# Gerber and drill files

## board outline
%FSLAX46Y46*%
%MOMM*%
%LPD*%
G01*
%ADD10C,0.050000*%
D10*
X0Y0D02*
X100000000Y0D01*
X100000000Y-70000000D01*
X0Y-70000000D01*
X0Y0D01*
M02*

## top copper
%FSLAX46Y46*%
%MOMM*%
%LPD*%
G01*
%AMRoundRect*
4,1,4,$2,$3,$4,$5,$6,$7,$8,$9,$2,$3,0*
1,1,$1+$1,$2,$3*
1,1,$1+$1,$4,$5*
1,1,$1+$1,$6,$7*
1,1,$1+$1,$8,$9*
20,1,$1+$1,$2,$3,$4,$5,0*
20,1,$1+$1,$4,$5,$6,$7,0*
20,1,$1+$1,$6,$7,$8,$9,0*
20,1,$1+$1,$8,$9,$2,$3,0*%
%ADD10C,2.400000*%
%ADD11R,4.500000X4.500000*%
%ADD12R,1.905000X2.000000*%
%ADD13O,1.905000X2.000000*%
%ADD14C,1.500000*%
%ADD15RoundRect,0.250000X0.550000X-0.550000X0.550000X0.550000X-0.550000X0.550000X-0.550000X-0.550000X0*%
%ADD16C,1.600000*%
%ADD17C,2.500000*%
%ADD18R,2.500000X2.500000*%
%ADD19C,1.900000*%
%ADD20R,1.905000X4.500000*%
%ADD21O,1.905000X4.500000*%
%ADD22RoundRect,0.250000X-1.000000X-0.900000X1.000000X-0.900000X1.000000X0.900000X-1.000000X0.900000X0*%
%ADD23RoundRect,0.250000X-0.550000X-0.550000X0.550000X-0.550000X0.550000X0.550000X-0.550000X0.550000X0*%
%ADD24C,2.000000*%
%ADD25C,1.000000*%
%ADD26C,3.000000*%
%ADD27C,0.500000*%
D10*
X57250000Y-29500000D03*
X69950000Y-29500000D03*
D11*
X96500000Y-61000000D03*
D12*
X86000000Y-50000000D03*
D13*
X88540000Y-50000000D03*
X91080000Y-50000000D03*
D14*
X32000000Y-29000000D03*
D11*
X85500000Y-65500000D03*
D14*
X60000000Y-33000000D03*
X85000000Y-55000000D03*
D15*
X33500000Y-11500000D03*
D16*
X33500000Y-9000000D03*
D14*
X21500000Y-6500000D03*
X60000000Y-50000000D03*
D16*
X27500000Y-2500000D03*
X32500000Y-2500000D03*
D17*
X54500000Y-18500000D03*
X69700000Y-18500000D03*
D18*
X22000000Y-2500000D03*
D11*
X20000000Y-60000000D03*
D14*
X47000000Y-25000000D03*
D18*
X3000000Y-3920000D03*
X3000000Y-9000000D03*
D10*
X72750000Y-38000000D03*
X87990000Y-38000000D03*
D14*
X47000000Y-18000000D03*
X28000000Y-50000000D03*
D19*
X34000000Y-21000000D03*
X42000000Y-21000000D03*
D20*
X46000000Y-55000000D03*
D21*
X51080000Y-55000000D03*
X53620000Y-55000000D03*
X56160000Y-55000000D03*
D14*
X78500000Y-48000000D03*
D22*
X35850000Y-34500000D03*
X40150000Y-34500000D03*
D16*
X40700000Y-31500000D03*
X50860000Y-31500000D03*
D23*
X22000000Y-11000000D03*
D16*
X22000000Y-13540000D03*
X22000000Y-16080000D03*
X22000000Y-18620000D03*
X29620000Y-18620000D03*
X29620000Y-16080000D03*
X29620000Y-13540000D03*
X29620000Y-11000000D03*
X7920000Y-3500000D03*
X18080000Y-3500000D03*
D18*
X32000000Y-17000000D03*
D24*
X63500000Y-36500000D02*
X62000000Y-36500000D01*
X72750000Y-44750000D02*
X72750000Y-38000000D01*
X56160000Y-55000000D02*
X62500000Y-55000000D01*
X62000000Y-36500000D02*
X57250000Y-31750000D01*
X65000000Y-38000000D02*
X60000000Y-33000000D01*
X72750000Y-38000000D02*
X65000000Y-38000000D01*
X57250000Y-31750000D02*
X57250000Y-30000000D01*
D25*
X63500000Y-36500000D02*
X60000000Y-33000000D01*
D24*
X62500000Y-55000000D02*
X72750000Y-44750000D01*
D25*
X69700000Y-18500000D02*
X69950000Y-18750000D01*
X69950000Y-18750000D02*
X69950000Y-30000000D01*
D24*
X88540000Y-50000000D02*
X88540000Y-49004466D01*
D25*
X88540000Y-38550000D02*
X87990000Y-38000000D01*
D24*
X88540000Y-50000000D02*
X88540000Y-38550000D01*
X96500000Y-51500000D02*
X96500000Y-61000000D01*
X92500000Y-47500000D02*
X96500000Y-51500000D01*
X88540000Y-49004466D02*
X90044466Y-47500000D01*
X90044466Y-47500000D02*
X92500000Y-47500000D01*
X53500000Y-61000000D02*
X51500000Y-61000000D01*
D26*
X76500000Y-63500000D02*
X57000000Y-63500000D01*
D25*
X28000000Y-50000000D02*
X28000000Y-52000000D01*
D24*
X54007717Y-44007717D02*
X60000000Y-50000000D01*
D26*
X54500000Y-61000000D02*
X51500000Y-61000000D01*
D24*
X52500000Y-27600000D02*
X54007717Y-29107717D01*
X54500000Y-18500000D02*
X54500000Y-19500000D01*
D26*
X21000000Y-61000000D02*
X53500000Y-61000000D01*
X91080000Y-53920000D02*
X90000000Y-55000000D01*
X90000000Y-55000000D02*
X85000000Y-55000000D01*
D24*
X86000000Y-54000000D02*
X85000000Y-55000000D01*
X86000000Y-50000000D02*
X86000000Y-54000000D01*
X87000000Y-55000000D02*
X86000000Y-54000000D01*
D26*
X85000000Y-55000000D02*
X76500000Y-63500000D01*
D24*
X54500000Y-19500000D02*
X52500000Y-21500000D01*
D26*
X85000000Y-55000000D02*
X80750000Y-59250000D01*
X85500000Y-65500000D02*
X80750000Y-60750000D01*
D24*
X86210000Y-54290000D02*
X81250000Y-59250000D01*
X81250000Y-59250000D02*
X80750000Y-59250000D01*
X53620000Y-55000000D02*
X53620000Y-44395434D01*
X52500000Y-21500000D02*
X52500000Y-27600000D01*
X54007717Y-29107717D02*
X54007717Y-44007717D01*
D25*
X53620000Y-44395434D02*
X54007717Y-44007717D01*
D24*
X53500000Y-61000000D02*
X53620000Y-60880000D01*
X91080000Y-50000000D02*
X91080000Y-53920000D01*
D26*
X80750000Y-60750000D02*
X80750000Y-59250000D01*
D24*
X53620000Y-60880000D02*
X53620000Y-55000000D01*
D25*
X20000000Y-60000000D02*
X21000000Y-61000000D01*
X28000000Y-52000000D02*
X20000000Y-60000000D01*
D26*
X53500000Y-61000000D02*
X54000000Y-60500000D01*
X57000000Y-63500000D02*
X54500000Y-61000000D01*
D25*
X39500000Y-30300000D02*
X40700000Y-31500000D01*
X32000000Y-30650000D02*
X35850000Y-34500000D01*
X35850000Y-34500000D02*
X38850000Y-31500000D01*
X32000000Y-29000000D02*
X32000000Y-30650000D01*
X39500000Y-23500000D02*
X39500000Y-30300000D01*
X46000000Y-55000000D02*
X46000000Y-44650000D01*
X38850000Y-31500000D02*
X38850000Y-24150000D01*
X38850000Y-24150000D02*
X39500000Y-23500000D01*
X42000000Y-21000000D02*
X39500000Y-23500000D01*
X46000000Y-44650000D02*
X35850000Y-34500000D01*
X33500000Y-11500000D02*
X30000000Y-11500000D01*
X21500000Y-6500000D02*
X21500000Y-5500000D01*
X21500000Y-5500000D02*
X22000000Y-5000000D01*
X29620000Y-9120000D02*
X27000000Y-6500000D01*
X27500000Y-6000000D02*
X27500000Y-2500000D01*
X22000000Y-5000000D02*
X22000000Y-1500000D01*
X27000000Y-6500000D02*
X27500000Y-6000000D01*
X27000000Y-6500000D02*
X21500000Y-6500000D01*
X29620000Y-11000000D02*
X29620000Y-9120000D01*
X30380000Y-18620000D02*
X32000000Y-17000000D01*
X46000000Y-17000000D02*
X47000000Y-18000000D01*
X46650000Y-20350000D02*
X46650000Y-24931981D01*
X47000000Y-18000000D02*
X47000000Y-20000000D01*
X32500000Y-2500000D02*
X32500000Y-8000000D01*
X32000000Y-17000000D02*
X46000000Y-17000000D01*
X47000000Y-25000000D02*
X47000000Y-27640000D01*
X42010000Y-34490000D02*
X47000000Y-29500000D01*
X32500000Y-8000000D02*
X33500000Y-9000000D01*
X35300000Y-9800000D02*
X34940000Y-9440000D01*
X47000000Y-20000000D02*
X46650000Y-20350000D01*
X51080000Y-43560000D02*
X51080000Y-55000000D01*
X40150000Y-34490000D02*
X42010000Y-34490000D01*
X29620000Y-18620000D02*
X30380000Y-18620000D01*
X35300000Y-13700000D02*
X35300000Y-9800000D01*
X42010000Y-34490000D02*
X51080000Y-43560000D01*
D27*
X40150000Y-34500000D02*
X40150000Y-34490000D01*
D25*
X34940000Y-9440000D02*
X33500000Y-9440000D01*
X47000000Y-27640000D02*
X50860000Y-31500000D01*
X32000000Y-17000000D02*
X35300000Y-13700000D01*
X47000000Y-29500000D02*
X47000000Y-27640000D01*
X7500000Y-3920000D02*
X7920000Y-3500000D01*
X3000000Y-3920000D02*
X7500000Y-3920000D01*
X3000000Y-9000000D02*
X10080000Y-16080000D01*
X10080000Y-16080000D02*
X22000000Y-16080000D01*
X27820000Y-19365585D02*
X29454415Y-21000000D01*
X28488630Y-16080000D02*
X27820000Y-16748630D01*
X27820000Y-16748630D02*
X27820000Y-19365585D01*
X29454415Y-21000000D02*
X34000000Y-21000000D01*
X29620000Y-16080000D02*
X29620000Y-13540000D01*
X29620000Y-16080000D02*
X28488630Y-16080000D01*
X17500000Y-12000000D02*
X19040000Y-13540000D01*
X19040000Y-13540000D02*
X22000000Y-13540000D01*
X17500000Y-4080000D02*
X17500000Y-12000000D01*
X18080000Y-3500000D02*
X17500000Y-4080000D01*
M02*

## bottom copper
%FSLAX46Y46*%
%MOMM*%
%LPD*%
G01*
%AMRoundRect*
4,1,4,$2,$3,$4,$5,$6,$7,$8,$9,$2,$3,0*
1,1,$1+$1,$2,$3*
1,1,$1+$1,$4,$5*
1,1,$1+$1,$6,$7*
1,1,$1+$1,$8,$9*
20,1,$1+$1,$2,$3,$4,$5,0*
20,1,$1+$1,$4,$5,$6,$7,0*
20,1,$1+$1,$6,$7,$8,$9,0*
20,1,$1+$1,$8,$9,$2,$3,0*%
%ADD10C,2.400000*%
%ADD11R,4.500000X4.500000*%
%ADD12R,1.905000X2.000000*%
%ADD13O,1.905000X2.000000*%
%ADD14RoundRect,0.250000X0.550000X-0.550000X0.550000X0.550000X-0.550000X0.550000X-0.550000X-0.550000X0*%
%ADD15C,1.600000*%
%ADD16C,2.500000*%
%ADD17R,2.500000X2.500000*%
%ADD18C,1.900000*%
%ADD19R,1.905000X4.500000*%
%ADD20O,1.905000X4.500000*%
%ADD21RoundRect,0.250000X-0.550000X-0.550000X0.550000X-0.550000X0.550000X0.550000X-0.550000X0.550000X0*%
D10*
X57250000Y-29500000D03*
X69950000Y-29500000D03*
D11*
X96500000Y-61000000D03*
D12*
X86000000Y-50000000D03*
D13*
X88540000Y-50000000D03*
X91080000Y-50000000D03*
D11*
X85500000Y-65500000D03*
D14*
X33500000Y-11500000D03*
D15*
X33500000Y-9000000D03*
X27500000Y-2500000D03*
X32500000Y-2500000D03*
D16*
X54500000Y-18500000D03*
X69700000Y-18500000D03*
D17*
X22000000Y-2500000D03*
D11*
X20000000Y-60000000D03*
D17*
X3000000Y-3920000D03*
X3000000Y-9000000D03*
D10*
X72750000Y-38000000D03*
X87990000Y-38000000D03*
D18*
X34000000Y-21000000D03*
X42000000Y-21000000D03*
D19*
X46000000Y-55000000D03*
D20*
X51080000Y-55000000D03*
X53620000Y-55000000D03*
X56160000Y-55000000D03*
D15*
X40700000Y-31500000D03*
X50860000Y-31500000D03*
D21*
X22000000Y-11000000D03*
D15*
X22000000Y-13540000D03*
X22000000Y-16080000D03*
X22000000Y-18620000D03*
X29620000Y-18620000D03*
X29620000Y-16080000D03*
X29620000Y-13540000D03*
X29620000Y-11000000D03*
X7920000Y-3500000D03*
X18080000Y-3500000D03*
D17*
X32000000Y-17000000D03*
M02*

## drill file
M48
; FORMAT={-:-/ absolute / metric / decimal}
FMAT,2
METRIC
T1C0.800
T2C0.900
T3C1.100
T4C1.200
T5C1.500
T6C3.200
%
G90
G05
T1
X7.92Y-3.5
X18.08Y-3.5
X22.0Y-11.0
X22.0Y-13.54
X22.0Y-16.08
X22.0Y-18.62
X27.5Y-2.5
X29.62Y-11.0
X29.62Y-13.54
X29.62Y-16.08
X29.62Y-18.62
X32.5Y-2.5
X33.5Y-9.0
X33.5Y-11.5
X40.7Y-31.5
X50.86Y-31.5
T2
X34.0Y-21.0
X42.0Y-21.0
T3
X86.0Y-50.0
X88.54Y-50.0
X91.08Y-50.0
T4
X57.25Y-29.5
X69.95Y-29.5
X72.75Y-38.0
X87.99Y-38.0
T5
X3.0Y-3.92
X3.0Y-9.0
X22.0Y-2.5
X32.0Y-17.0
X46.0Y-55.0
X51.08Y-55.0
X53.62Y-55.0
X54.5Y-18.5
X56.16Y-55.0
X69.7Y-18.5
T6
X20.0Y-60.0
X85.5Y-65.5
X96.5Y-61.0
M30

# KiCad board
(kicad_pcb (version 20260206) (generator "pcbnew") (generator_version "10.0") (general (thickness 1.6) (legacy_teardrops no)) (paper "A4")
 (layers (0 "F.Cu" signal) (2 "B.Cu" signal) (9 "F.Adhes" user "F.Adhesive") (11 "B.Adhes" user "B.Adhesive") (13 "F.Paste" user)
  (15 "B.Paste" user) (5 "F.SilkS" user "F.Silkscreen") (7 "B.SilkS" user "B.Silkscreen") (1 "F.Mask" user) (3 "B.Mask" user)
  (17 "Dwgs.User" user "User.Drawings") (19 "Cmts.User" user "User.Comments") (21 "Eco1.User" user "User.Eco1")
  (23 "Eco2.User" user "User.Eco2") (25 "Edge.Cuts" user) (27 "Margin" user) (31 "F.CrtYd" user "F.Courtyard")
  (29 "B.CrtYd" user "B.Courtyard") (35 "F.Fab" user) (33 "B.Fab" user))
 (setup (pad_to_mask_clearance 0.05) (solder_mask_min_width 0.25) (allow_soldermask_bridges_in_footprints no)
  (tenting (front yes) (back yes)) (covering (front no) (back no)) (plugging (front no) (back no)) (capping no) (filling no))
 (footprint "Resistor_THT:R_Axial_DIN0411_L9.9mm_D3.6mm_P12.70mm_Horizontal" (layer "F.Cu") (at 57.25 29.5)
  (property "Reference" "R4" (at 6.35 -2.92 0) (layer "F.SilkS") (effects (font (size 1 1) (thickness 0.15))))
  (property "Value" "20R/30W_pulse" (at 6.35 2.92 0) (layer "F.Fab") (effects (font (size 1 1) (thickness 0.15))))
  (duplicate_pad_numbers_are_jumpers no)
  (pad "1" thru_hole circle (at 0 0) (size 2.4 2.4) (drill 1.2) (layers "*.Cu" "*.Mask") (remove_unused_layers no) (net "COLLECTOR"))
  (pad "2" thru_hole circle (at 12.7 0) (size 2.4 2.4) (drill 1.2) (layers "*.Cu" "*.Mask") (remove_unused_layers no)
   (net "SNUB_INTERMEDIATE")))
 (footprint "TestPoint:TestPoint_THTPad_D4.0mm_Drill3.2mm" (layer "F.Cu") (at 96.5 61)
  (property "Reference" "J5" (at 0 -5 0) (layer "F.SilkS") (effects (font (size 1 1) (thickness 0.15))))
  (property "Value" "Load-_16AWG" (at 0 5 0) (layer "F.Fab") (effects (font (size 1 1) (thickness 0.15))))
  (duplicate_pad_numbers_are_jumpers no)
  (pad "1" thru_hole rect (at 0 0) (size 4.5 4.5) (drill 3.2) (layers "*.Cu" "*.Mask") (remove_unused_layers no) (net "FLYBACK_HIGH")))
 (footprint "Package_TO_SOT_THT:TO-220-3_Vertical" (layer "F.Cu") (at 86 50)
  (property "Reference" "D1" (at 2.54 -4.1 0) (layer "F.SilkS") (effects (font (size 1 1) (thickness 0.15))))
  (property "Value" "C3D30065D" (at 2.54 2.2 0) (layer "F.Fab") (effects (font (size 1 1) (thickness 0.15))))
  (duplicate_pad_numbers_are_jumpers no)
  (pad "1" thru_hole rect (at 0 0) (size 1.905 2) (drill 1.1) (layers "*.Cu" "*.Mask") (remove_unused_layers no) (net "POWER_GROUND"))
  (pad "2" thru_hole oval (at 2.54 0) (size 1.905 2) (drill 1.1) (layers "*.Cu" "*.Mask") (remove_unused_layers no) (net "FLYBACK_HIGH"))
  (pad "3" thru_hole oval (at 5.08 0) (size 1.905 2) (drill 1.1) (layers "*.Cu" "*.Mask") (remove_unused_layers no) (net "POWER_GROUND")))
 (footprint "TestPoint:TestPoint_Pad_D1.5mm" (layer "F.Cu") (at 32 29)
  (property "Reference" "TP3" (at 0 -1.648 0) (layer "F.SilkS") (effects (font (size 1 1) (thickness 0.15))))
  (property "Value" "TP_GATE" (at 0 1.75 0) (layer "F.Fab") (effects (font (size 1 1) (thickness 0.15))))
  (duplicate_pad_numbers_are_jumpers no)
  (pad "1" smd circle (at 0 0) (size 1.5 1.5) (layers "F.Cu" "F.Mask") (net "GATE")))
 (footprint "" (layer "F.Cu") (at 85.5 65.5)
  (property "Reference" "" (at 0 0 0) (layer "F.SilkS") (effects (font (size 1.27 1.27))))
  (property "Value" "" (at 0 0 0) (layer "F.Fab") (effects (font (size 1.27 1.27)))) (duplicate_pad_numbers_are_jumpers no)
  (pad "1" thru_hole rect (at 0 0) (size 4.5 4.5) (drill 3.2) (layers "*.Cu" "*.Mask") (remove_unused_layers no) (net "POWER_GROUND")))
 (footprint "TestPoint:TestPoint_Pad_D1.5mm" (layer "F.Cu") (at 60 33)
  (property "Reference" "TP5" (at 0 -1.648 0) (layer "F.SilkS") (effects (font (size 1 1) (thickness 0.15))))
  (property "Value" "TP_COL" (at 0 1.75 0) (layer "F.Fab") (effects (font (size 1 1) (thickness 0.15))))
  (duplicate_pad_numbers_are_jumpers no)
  (pad "1" smd circle (at 0 0) (size 1.5 1.5) (layers "F.Cu" "F.Mask") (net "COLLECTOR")))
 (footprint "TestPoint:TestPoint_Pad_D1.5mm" (layer "F.Cu") (at 85 55)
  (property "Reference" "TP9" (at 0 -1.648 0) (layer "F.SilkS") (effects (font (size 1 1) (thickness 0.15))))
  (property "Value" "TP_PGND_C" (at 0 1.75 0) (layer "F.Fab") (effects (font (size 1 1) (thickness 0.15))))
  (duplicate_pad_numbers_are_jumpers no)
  (pad "1" smd circle (at 0 0) (size 1.5 1.5) (layers "F.Cu" "F.Mask") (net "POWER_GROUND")))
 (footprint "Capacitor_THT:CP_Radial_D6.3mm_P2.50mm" (layer "F.Cu") (at 33.5 11.5 90)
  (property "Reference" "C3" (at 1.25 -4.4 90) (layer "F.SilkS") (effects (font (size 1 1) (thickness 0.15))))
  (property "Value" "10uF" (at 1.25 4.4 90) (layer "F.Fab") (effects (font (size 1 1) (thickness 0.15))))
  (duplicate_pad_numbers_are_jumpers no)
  (pad "1" thru_hole roundrect (at 0 0 90) (size 1.6 1.6) (drill 0.8) (layers "*.Cu" "*.Mask") (remove_unused_layers no)
   (roundrect_rratio 0.15625) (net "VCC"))
  (pad "2" thru_hole circle (at 2.5 0 90) (size 1.6 1.6) (drill 0.8) (layers "*.Cu" "*.Mask") (remove_unused_layers no)
   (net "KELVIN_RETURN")))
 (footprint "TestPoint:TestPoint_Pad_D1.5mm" (layer "F.Cu") (at 21.5 6.5)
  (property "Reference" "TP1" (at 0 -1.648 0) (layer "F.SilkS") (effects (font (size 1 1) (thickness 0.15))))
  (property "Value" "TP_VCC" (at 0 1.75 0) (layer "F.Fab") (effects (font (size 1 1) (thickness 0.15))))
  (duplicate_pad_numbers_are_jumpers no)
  (pad "1" smd circle (at 0 0) (size 1.5 1.5) (layers "F.Cu" "F.Mask") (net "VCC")))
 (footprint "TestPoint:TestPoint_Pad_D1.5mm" (layer "F.Cu") (at 60 50)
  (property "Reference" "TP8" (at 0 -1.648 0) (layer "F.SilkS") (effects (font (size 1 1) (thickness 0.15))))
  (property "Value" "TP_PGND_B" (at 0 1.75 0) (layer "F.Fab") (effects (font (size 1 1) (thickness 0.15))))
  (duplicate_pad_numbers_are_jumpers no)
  (pad "1" smd circle (at 0 0) (size 1.5 1.5) (layers "F.Cu" "F.Mask") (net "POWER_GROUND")))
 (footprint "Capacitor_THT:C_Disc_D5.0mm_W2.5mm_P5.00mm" (layer "F.Cu") (at 27.5 2.5)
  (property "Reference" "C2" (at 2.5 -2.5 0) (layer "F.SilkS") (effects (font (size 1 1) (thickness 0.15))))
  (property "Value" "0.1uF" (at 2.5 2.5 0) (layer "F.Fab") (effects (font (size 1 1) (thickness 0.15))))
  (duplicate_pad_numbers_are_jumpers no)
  (pad "1" thru_hole circle (at 0 0) (size 1.6 1.6) (drill 0.8) (layers "*.Cu" "*.Mask") (remove_unused_layers no) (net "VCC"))
  (pad "2" thru_hole circle (at 5 0) (size 1.6 1.6) (drill 0.8) (layers "*.Cu" "*.Mask") (remove_unused_layers no) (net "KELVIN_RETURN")))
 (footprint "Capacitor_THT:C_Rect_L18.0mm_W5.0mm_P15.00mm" (layer "F.Cu") (at 62.1 18.5)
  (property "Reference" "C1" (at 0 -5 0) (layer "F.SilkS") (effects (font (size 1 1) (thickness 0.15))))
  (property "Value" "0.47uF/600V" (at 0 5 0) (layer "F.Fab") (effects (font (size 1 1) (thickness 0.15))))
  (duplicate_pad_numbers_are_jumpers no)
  (pad "1" thru_hole circle (at -7.6 0) (size 2.5 2.5) (drill 1.5) (layers "*.Cu" "*.Mask") (remove_unused_layers no) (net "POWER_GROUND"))
  (pad "2" thru_hole circle (at 7.6 0) (size 2.5 2.5) (drill 1.5) (layers "*.Cu" "*.Mask") (remove_unused_layers no)
   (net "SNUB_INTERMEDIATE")))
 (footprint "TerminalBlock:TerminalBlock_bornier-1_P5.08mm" (layer "F.Cu") (at 22 2.5)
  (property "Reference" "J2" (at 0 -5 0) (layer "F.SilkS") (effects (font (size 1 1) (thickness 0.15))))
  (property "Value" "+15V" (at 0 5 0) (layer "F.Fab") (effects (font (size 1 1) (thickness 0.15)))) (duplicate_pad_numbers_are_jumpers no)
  (pad "1" thru_hole rect (at 0 0) (size 2.5 2.5) (drill 1.5) (layers "*.Cu" "*.Mask") (remove_unused_layers no) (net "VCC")))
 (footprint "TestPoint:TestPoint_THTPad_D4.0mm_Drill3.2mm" (layer "F.Cu") (at 20 60)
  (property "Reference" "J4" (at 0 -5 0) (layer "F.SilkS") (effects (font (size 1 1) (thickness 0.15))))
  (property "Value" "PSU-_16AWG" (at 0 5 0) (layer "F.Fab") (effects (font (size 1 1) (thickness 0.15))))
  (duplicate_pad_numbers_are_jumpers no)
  (pad "1" thru_hole rect (at 0 0) (size 4.5 4.5) (drill 3.2) (layers "*.Cu" "*.Mask") (remove_unused_layers no) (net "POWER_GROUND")))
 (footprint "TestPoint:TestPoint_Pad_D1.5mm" (layer "F.Cu") (at 47 25)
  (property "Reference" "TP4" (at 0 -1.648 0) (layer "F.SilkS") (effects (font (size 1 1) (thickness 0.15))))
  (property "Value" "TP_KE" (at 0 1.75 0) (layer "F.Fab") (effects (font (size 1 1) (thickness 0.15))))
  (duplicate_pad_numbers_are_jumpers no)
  (pad "1" smd circle (at 0 0) (size 1.5 1.5) (layers "F.Cu" "F.Mask") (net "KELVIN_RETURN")))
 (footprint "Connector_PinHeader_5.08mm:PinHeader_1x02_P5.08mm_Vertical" (layer "F.Cu") (at 3 6.46)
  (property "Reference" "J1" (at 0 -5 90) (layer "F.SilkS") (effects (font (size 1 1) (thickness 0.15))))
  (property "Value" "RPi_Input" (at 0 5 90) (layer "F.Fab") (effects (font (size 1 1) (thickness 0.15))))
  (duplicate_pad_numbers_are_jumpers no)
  (pad "1" thru_hole rect (at 0 -2.54 270) (size 2.5 2.5) (drill 1.5) (layers "*.Cu" "*.Mask") (remove_unused_layers no) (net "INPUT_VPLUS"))
  (pad "2" thru_hole rect (at 0 2.54 270) (size 2.5 2.5) (drill 1.5) (layers "*.Cu" "*.Mask") (remove_unused_layers no) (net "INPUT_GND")))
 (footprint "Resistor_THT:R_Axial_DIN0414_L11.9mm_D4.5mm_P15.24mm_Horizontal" (layer "F.Cu") (at 72.75 38)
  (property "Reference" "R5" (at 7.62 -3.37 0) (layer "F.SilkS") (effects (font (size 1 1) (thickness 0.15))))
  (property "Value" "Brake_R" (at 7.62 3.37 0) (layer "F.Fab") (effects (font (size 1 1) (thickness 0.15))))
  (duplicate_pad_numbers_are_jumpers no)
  (pad "1" thru_hole circle (at 0 0) (size 2.4 2.4) (drill 1.2) (layers "*.Cu" "*.Mask") (remove_unused_layers no) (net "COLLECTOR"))
  (pad "2" thru_hole circle (at 15.24 0) (size 2.4 2.4) (drill 1.2) (layers "*.Cu" "*.Mask") (remove_unused_layers no) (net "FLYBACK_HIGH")))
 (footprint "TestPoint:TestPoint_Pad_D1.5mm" (layer "F.Cu") (at 47 18)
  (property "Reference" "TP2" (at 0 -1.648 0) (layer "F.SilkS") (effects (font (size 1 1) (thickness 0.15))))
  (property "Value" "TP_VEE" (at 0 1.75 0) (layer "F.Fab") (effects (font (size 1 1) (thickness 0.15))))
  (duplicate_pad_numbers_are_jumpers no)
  (pad "1" smd circle (at 0 0) (size 1.5 1.5) (layers "F.Cu" "F.Mask") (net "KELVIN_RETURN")))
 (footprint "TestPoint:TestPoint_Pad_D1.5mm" (layer "F.Cu") (at 28 50)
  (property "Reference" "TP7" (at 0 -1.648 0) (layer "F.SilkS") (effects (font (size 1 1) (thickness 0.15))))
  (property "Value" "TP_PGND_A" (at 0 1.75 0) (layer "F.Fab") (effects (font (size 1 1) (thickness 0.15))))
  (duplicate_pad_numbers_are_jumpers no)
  (pad "1" smd circle (at 0 0) (size 1.5 1.5) (layers "F.Cu" "F.Mask") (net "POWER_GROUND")))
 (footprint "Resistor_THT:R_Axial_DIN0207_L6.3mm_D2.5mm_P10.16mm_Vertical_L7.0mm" (layer "F.Cu") (at 38 21 90)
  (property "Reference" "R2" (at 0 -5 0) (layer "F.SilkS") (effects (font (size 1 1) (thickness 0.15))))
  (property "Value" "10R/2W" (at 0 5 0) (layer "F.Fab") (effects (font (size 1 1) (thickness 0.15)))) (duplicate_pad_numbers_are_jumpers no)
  (pad "1" thru_hole circle (at 0 -4) (size 1.9 1.9) (drill 0.9) (layers "*.Cu" "*.Mask") (remove_unused_layers no) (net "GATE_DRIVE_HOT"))
  (pad "2" thru_hole circle (at 0 4) (size 1.9 1.9) (drill 0.9) (layers "*.Cu" "*.Mask") (remove_unused_layers no) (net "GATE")))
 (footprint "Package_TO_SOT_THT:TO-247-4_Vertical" (layer "F.Cu") (at 46 55)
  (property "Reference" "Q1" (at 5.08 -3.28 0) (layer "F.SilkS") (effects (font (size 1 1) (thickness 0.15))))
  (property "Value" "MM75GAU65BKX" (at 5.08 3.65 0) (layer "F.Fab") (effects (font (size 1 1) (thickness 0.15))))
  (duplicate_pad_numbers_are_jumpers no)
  (pad "1" thru_hole rect (at 0 0) (size 1.905 4.5) (drill 1.5) (layers "*.Cu" "*.Mask") (remove_unused_layers no) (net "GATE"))
  (pad "2" thru_hole oval (at 5.08 0) (size 1.905 4.5) (drill 1.5) (layers "*.Cu" "*.Mask") (remove_unused_layers no) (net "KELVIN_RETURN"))
  (pad "3" thru_hole oval (at 7.62 0) (size 1.905 4.5) (drill 1.5) (layers "*.Cu" "*.Mask") (remove_unused_layers no) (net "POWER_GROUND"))
  (pad "4" thru_hole oval (at 10.16 0) (size 1.905 4.5) (drill 1.5) (layers "*.Cu" "*.Mask") (remove_unused_layers no) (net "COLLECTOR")))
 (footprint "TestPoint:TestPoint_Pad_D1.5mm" (layer "F.Cu") (at 78.5 48)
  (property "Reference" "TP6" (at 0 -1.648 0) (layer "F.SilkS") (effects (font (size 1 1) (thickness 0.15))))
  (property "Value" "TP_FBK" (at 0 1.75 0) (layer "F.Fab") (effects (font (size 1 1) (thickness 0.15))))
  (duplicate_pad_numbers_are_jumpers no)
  (pad "1" smd circle (at 0 0) (size 1.5 1.5) (layers "F.Cu" "F.Mask") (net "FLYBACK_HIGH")))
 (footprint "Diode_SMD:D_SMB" (layer "F.Cu") (at 38 34.5)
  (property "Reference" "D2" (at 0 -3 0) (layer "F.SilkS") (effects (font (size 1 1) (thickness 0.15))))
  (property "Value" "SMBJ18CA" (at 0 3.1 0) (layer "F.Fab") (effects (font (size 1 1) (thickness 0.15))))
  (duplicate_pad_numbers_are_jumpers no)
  (pad "1" smd roundrect (at -2.15 0) (size 2.5 2.3) (layers "F.Cu" "F.Mask" "F.Paste") (roundrect_rratio 0.1086956522) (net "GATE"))
  (pad "2" smd roundrect (at 2.15 0) (size 2.5 2.3) (layers "F.Cu" "F.Mask" "F.Paste") (roundrect_rratio 0.1086956522) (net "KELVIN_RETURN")))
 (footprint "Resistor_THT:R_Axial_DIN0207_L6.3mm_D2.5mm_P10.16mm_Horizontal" (layer "F.Cu") (at 40.7 31.5)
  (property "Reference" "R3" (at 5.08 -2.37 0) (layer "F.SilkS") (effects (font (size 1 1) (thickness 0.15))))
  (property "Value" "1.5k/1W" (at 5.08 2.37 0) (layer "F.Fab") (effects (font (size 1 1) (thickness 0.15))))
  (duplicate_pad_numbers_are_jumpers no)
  (pad "1" thru_hole circle (at 0 0) (size 1.6 1.6) (drill 0.8) (layers "*.Cu" "*.Mask") (remove_unused_layers no) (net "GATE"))
  (pad "2" thru_hole circle (at 10.16 0) (size 1.6 1.6) (drill 0.8) (layers "*.Cu" "*.Mask") (remove_unused_layers no) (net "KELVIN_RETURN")))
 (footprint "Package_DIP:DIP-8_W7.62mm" (layer "F.Cu") (at 22 11)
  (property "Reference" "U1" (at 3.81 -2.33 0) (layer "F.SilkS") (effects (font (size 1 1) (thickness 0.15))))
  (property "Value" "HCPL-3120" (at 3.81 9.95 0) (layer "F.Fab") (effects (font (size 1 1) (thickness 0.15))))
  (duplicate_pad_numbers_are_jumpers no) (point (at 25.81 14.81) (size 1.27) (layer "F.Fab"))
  (pad "1" thru_hole roundrect (at 0 0) (size 1.6 1.6) (drill 0.8) (layers "*.Cu" "*.Mask") (remove_unused_layers no)
   (roundrect_rratio 0.15625))
  (pad "2" thru_hole circle (at 0 2.54) (size 1.6 1.6) (drill 0.8) (layers "*.Cu" "*.Mask") (remove_unused_layers no) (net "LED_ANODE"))
  (pad "3" thru_hole circle (at 0 5.08) (size 1.6 1.6) (drill 0.8) (layers "*.Cu" "*.Mask") (remove_unused_layers no) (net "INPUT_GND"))
  (pad "4" thru_hole circle (at 0 7.62) (size 1.6 1.6) (drill 0.8) (layers "*.Cu" "*.Mask") (remove_unused_layers no))
  (pad "5" thru_hole circle (at 7.62 7.62) (size 1.6 1.6) (drill 0.8) (layers "*.Cu" "*.Mask") (remove_unused_layers no)
   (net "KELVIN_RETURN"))
  (pad "6" thru_hole circle (at 7.62 5.08) (size 1.6 1.6) (drill 0.8) (layers "*.Cu" "*.Mask") (remove_unused_layers no)
   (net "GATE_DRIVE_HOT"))
  (pad "7" thru_hole circle (at 7.62 2.54) (size 1.6 1.6) (drill 0.8) (layers "*.Cu" "*.Mask") (remove_unused_layers no)
   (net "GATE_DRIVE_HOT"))
  (pad "8" thru_hole circle (at 7.62 0) (size 1.6 1.6) (drill 0.8) (layers "*.Cu" "*.Mask") (remove_unused_layers no) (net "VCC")))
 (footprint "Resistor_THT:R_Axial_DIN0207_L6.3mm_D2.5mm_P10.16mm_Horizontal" (layer "F.Cu") (at 7.92 3.5)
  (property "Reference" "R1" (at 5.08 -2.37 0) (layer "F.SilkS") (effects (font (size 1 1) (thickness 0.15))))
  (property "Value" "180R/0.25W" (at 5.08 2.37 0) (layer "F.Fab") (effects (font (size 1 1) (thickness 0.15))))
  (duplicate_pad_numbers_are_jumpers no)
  (pad "1" thru_hole circle (at 0 0) (size 1.6 1.6) (drill 0.8) (layers "*.Cu" "*.Mask") (remove_unused_layers no) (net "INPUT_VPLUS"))
  (pad "2" thru_hole circle (at 10.16 0) (size 1.6 1.6) (drill 0.8) (layers "*.Cu" "*.Mask") (remove_unused_layers no) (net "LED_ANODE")))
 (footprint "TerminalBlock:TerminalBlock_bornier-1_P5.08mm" (layer "F.Cu") (at 32 17)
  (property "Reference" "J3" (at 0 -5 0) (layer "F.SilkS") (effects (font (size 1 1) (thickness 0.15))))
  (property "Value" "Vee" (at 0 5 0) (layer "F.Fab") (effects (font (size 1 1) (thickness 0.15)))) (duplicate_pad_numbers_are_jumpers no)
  (pad "1" thru_hole rect (at 0 0) (size 2.5 2.5) (drill 1.5) (layers "*.Cu" "*.Mask") (remove_unused_layers no) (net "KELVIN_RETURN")))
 (gr_rect (start 0 0) (end 100 70) (stroke (width 0.05) (type solid)) (fill no) (layer "Edge.Cuts"))
 (segment (start 63.5 36.5) (end 62 36.5) (width 2) (layer "F.Cu") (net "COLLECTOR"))
 (segment (start 72.75 44.75) (end 72.75 38) (width 2) (layer "F.Cu") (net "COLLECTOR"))
 (segment (start 56.16 55) (end 62.5 55) (width 2) (layer "F.Cu") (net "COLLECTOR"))
 (segment (start 62 36.5) (end 57.25 31.75) (width 2) (layer "F.Cu") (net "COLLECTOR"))
 (segment (start 65 38) (end 60 33) (width 2) (layer "F.Cu") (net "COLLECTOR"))
 (segment (start 72.75 38) (end 65 38) (width 2) (layer "F.Cu") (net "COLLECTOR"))
 (segment (start 57.25 31.75) (end 57.25 30) (width 2) (layer "F.Cu") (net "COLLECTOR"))
 (segment (start 63.5 36.5) (end 60 33) (width 1) (layer "F.Cu") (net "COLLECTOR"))
 (segment (start 62.5 55) (end 72.75 44.75) (width 2) (layer "F.Cu") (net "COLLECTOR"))
 (segment (start 69.7 18.5) (end 69.95 18.75) (width 1) (layer "F.Cu") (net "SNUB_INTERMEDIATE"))
 (segment (start 69.95 18.75) (end 69.95 30) (width 1) (layer "F.Cu") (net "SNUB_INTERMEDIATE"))
 (segment (start 88.54 50) (end 88.54 49.004466) (width 2) (layer "F.Cu") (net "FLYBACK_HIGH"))
 (segment (start 88.54 38.55) (end 87.99 38) (width 1) (layer "F.Cu") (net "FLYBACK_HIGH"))
 (segment (start 88.54 50) (end 88.54 38.55) (width 2) (layer "F.Cu") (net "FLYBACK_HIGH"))
 (segment (start 96.5 51.5) (end 96.5 61) (width 2) (layer "F.Cu") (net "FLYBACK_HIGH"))
 (segment (start 92.5 47.5) (end 96.5 51.5) (width 2) (layer "F.Cu") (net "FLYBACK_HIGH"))
 (segment (start 88.54 49.004466) (end 90.044466 47.5) (width 2) (layer "F.Cu") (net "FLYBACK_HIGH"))
 (segment (start 90.044466 47.5) (end 92.5 47.5) (width 2) (layer "F.Cu") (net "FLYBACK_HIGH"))
 (segment (start 53.5 61) (end 51.5 61) (width 2) (layer "F.Cu") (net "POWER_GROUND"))
 (segment (start 76.5 63.5) (end 57 63.5) (width 3) (layer "F.Cu") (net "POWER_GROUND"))
 (segment (start 28 50) (end 28 52) (width 1) (layer "F.Cu") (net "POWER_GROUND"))
 (segment (start 54.007717 44.007717) (end 60 50) (width 2) (layer "F.Cu") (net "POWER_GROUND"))
 (segment (start 54.5 61) (end 51.5 61) (width 3) (layer "F.Cu") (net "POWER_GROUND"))
 (segment (start 52.5 27.6) (end 54.007717 29.107717) (width 2) (layer "F.Cu") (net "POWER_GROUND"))
 (segment (start 54.5 18.5) (end 54.5 19.5) (width 2) (layer "F.Cu") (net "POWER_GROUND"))
 (segment (start 21 61) (end 53.5 61) (width 3) (layer "F.Cu") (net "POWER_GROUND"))
 (segment (start 91.08 53.92) (end 90 55) (width 3) (layer "F.Cu") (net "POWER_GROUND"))
 (segment (start 90 55) (end 85 55) (width 3) (layer "F.Cu") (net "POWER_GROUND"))
 (segment (start 86 54) (end 85 55) (width 2) (layer "F.Cu") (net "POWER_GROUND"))
 (segment (start 86 50) (end 86 54) (width 2) (layer "F.Cu") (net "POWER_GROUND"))
 (segment (start 87 55) (end 86 54) (width 2) (layer "F.Cu") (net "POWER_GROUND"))
 (segment (start 85 55) (end 76.5 63.5) (width 3) (layer "F.Cu") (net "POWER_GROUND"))
 (segment (start 54.5 19.5) (end 52.5 21.5) (width 2) (layer "F.Cu") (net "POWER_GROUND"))
 (segment (start 85 55) (end 80.75 59.25) (width 3) (layer "F.Cu") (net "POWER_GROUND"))
 (segment (start 85.5 65.5) (end 80.75 60.75) (width 3) (layer "F.Cu") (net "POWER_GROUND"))
 (segment (start 86.21 54.29) (end 81.25 59.25) (width 2) (layer "F.Cu") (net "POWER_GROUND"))
 (segment (start 81.25 59.25) (end 80.75 59.25) (width 2) (layer "F.Cu") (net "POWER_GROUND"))
 (segment (start 53.62 55) (end 53.62 44.395434) (width 2) (layer "F.Cu") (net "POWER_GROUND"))
 (segment (start 52.5 21.5) (end 52.5 27.6) (width 2) (layer "F.Cu") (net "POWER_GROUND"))
 (segment (start 54.007717 29.107717) (end 54.007717 44.007717) (width 2) (layer "F.Cu") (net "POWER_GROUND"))
 (segment (start 53.62 44.395434) (end 54.007717 44.007717) (width 1) (layer "F.Cu") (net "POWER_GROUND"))
 (segment (start 53.5 61) (end 53.62 60.88) (width 2) (layer "F.Cu") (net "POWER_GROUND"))
 (segment (start 91.08 50) (end 91.08 53.92) (width 2) (layer "F.Cu") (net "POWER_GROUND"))
 (segment (start 80.75 60.75) (end 80.75 59.25) (width 3) (layer "F.Cu") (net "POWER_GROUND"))
 (segment (start 53.62 60.88) (end 53.62 55) (width 2) (layer "F.Cu") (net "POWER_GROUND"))
 (segment (start 20 60) (end 21 61) (width 1) (layer "F.Cu") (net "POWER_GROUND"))
 (segment (start 28 52) (end 20 60) (width 1) (layer "F.Cu") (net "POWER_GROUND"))
 (segment (start 53.5 61) (end 54 60.5) (width 3) (layer "F.Cu") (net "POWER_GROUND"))
 (segment (start 57 63.5) (end 54.5 61) (width 3) (layer "F.Cu") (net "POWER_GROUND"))
 (segment (start 39.5 30.3) (end 40.7 31.5) (width 1) (layer "F.Cu") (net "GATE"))
 (segment (start 32 30.65) (end 35.85 34.5) (width 1) (layer "F.Cu") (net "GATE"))
 (segment (start 35.85 34.5) (end 38.85 31.5) (width 1) (layer "F.Cu") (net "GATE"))
 (segment (start 32 29) (end 32 30.65) (width 1) (layer "F.Cu") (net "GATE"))
 (segment (start 39.5 23.5) (end 39.5 30.3) (width 1) (layer "F.Cu") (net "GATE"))
 (segment (start 46 55) (end 46 44.65) (width 1) (layer "F.Cu") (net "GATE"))
 (segment (start 38.85 31.5) (end 38.85 24.15) (width 1) (layer "F.Cu") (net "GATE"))
 (segment (start 38.85 24.15) (end 39.5 23.5) (width 1) (layer "F.Cu") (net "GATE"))
 (segment (start 42 21) (end 39.5 23.5) (width 1) (layer "F.Cu") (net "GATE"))
 (segment (start 46 44.65) (end 35.85 34.5) (width 1) (layer "F.Cu") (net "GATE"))
 (segment (start 33.5 11.5) (end 30 11.5) (width 1) (layer "F.Cu") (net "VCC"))
 (segment (start 21.5 6.5) (end 21.5 5.5) (width 1) (layer "F.Cu") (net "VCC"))
 (segment (start 21.5 5.5) (end 22 5) (width 1) (layer "F.Cu") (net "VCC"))
 (segment (start 29.62 9.12) (end 27 6.5) (width 1) (layer "F.Cu") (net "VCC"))
 (segment (start 27.5 6) (end 27.5 2.5) (width 1) (layer "F.Cu") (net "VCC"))
 (segment (start 22 5) (end 22 1.5) (width 1) (layer "F.Cu") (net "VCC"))
 (segment (start 27 6.5) (end 27.5 6) (width 1) (layer "F.Cu") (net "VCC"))
 (segment (start 27 6.5) (end 21.5 6.5) (width 1) (layer "F.Cu") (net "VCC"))
 (segment (start 29.62 11) (end 29.62 9.12) (width 1) (layer "F.Cu") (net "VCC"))
 (segment (start 30.38 18.62) (end 32 17) (width 1) (layer "F.Cu") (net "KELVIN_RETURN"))
 (segment (start 46 17) (end 47 18) (width 1) (layer "F.Cu") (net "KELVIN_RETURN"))
 (segment (start 46.65 20.35) (end 46.65 24.931981) (width 1) (layer "F.Cu") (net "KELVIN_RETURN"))
 (segment (start 47 18) (end 47 20) (width 1) (layer "F.Cu") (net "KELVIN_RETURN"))
 (segment (start 32.5 2.5) (end 32.5 8) (width 1) (layer "F.Cu") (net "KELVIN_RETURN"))
 (segment (start 32 17) (end 46 17) (width 1) (layer "F.Cu") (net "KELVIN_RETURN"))
 (segment (start 47 25) (end 47 27.64) (width 1) (layer "F.Cu") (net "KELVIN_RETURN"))
 (segment (start 42.01 34.49) (end 47 29.5) (width 1) (layer "F.Cu") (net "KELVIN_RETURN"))
 (segment (start 32.5 8) (end 33.5 9) (width 1) (layer "F.Cu") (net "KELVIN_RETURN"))
 (segment (start 35.3 9.8) (end 34.94 9.44) (width 1) (layer "F.Cu") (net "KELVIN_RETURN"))
 (segment (start 47 20) (end 46.65 20.35) (width 1) (layer "F.Cu") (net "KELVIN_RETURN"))
 (segment (start 51.08 43.56) (end 51.08 55) (width 1) (layer "F.Cu") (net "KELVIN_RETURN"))
 (segment (start 40.15 34.49) (end 42.01 34.49) (width 1) (layer "F.Cu") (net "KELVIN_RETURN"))
 (segment (start 29.62 18.62) (end 30.38 18.62) (width 1) (layer "F.Cu") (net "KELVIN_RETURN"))
 (segment (start 35.3 13.7) (end 35.3 9.8) (width 1) (layer "F.Cu") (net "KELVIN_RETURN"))
 (segment (start 42.01 34.49) (end 51.08 43.56) (width 1) (layer "F.Cu") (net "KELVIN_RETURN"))
 (segment (start 40.15 34.5) (end 40.15 34.49) (width 0.5) (layer "F.Cu") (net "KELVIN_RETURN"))
 (segment (start 34.94 9.44) (end 33.5 9.44) (width 1) (layer "F.Cu") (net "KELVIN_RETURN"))
 (segment (start 47 27.64) (end 50.86 31.5) (width 1) (layer "F.Cu") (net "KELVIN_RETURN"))
 (segment (start 32 17) (end 35.3 13.7) (width 1) (layer "F.Cu") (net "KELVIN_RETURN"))
 (segment (start 47 29.5) (end 47 27.64) (width 1) (layer "F.Cu") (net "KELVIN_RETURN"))
 (segment (start 7.5 3.92) (end 7.92 3.5) (width 1) (layer "F.Cu") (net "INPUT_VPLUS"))
 (segment (start 3 3.92) (end 7.5 3.92) (width 1) (layer "F.Cu") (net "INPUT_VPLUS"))
 (segment (start 3 9) (end 10.08 16.08) (width 1) (layer "F.Cu") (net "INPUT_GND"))
 (segment (start 10.08 16.08) (end 22 16.08) (width 1) (layer "F.Cu") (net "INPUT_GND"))
 (segment (start 27.82 19.365585) (end 29.454415 21) (width 1) (layer "F.Cu") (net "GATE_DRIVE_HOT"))
 (segment (start 28.48863 16.08) (end 27.82 16.74863) (width 1) (layer "F.Cu") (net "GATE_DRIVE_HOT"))
 (segment (start 27.82 16.74863) (end 27.82 19.365585) (width 1) (layer "F.Cu") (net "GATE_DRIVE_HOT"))
 (segment (start 29.454415 21) (end 34 21) (width 1) (layer "F.Cu") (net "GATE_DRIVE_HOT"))
 (segment (start 29.62 16.08) (end 29.62 13.54) (width 1) (layer "F.Cu") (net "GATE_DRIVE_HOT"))
 (segment (start 29.62 16.08) (end 28.48863 16.08) (width 1) (layer "F.Cu") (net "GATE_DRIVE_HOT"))
 (segment (start 17.5 12) (end 19.04 13.54) (width 1) (layer "F.Cu") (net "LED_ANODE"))
 (segment (start 19.04 13.54) (end 22 13.54) (width 1) (layer "F.Cu") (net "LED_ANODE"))
 (segment (start 17.5 4.08) (end 17.5 12) (width 1) (layer "F.Cu") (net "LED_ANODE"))
 (segment (start 18.08 3.5) (end 17.5 4.08) (width 1) (layer "F.Cu") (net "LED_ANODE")))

